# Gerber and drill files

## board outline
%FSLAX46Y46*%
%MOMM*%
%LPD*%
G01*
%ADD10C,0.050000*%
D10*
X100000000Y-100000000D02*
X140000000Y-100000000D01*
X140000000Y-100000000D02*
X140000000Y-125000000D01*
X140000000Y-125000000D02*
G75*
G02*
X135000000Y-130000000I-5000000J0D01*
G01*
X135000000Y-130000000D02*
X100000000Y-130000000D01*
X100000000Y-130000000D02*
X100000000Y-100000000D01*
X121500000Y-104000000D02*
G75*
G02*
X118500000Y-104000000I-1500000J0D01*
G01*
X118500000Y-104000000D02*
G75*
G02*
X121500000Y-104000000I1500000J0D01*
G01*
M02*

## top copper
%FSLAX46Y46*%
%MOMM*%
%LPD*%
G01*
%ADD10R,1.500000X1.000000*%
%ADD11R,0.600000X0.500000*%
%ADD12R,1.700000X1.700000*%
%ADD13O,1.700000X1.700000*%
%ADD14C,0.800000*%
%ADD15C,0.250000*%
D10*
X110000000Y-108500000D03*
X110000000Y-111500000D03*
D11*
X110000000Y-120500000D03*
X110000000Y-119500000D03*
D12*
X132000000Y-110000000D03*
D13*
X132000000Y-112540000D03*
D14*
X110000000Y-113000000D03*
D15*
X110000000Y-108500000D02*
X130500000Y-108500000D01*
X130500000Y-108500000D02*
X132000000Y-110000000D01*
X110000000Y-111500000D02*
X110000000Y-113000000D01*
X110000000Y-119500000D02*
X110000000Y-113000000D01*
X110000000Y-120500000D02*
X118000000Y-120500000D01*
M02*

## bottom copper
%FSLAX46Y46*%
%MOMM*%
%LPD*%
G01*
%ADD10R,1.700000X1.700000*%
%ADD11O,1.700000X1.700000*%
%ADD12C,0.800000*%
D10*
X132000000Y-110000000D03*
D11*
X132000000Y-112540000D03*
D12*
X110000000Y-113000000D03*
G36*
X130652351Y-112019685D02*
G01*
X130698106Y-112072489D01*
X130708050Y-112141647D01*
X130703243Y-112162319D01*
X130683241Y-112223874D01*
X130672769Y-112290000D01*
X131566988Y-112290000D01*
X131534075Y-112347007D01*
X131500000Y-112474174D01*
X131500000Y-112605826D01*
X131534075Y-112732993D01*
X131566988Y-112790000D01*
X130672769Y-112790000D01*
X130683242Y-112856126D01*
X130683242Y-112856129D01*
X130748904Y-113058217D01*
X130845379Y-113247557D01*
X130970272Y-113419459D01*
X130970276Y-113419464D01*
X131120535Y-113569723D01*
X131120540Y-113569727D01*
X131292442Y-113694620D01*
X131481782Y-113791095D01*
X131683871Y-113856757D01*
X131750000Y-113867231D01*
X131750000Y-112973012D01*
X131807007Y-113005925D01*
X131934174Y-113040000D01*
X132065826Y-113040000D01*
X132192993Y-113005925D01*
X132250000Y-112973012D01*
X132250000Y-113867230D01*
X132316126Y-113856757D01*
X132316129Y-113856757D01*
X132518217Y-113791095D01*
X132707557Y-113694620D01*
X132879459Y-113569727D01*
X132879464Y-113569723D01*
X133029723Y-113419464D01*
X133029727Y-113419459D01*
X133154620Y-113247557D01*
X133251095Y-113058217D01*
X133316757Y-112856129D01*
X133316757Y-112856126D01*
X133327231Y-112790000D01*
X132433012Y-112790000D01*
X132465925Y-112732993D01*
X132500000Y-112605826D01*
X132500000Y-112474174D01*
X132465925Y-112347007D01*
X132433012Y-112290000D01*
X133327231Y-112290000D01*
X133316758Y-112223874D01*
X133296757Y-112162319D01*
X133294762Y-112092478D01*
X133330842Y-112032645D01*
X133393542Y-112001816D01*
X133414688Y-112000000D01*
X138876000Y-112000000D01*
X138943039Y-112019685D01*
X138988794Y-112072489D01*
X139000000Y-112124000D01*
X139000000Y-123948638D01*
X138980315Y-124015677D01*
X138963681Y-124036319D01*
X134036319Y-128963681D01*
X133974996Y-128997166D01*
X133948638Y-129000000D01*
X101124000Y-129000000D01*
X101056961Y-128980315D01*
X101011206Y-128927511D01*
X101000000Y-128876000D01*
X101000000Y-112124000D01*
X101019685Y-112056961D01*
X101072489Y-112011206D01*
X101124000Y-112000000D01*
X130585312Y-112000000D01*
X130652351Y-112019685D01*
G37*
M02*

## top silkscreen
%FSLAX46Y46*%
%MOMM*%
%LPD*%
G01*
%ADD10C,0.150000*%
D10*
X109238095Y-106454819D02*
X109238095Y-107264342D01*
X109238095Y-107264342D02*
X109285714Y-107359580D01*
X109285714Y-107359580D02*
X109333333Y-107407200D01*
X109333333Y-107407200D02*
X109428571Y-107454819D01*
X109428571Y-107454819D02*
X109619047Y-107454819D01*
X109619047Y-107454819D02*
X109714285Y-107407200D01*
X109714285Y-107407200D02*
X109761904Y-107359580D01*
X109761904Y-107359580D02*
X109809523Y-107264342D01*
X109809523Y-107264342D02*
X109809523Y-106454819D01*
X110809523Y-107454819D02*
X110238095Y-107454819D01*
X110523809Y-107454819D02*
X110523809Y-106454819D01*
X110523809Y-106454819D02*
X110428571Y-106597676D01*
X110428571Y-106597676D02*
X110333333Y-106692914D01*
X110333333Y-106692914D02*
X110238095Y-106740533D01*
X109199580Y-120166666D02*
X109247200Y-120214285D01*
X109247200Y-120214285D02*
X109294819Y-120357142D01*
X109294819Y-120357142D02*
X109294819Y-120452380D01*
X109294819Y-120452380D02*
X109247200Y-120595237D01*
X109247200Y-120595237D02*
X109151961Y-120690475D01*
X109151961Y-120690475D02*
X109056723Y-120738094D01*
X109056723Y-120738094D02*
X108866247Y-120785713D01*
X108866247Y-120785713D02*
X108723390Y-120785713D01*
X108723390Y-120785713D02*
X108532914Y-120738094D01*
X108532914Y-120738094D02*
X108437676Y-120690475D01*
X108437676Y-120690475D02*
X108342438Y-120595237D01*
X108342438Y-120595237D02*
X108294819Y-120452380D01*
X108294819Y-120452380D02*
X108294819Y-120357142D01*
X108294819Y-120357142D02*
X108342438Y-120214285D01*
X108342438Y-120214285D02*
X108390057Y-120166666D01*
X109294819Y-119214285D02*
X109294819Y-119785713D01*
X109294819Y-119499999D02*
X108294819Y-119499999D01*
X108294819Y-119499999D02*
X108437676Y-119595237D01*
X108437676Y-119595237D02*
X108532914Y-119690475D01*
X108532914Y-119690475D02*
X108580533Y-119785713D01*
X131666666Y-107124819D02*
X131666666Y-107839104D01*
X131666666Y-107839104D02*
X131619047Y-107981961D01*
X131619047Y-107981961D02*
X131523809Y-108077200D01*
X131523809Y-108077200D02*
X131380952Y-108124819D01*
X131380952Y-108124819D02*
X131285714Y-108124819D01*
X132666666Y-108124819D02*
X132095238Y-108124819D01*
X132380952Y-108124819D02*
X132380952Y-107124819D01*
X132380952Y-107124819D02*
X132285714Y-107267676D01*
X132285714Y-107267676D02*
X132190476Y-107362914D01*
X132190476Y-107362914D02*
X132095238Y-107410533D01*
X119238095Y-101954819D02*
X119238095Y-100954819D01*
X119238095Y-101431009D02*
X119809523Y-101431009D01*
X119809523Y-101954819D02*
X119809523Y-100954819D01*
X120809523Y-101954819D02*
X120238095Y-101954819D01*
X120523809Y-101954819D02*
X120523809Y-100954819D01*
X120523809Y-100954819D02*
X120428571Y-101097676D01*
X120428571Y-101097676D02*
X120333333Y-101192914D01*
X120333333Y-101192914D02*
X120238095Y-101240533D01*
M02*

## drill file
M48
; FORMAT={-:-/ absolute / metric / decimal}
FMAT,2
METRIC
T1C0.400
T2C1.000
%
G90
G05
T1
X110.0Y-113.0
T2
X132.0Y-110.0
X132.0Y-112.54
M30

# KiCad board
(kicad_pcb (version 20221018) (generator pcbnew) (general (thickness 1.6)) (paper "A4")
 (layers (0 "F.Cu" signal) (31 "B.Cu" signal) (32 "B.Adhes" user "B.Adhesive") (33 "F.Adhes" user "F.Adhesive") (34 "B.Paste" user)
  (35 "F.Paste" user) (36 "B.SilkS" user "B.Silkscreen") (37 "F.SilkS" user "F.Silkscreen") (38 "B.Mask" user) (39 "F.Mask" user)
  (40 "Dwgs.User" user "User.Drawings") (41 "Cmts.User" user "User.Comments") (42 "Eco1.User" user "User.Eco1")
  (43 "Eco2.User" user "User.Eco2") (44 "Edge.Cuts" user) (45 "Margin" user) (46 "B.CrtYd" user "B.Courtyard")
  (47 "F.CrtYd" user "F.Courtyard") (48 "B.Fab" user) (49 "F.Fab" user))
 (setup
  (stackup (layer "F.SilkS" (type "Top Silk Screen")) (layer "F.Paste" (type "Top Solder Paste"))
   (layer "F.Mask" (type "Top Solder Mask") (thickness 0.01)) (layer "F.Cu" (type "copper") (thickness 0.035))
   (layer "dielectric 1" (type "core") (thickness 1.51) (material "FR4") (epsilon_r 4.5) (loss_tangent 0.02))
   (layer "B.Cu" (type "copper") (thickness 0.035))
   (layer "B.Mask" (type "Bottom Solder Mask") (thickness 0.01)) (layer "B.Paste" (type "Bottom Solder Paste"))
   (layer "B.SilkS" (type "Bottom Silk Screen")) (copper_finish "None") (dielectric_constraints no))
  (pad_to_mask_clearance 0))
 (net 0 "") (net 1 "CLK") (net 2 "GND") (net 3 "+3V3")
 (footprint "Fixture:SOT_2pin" (layer "F.Cu") (at 110 110)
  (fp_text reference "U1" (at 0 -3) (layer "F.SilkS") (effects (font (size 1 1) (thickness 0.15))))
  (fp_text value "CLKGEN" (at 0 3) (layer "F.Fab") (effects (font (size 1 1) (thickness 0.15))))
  (pad "1" smd rect (at 0 -1.5) (size 1.5 1) (layers "F.Cu" "F.Paste" "F.Mask") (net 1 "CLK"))
  (pad "2" smd rect (at 0 1.5) (size 1.5 1) (layers "F.Cu" "F.Paste" "F.Mask") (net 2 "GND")))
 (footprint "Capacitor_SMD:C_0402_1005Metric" (layer "F.Cu") (at 110 120 90)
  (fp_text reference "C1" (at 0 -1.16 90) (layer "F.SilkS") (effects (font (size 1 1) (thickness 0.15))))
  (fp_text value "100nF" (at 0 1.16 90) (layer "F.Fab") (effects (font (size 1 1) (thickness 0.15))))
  (pad "1" smd rect (at -0.5 0 90) (size 0.5 0.6) (layers "F.Cu" "F.Paste" "F.Mask") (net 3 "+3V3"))
  (pad "2" smd rect (at 0.5 0 90) (size 0.5 0.6) (layers "F.Cu" "F.Paste" "F.Mask") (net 2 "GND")))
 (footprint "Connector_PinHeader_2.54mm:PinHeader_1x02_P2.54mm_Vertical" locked (layer "F.Cu") (at 132 110)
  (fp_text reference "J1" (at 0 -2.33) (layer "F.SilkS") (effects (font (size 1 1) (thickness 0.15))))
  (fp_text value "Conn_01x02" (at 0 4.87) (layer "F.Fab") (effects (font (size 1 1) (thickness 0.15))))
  (pad "1" thru_hole rect (at 0 0) (size 1.7 1.7) (drill 1) (layers "*.Cu" "*.Mask") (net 1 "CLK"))
  (pad "2" thru_hole oval (at 0 2.54) (size 1.7 1.7) (drill 1) (layers "*.Cu" "*.Mask") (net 2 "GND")))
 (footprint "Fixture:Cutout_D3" (layer "F.Cu") (at 120 104)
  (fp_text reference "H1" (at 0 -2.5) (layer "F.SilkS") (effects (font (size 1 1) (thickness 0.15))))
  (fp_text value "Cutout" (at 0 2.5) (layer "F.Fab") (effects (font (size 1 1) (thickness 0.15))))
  (fp_circle (center 0 0) (end 1.5 0) (stroke (width 0.05) (type default)) (fill none) (layer "Edge.Cuts")))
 (gr_line (start 100 100) (end 140 100) (stroke (width 0.05) (type default)) (layer "Edge.Cuts"))
 (gr_line (start 140 100) (end 140 125) (stroke (width 0.05) (type default)) (layer "Edge.Cuts"))
 (gr_arc (start 140 125) (mid 138.535534 128.535534) (end 135 130) (stroke (width 0.05) (type default)) (layer "Edge.Cuts"))
 (gr_line (start 135 130) (end 100 130) (stroke (width 0.05) (type default)) (layer "Edge.Cuts"))
 (gr_line (start 100 130) (end 100 100) (stroke (width 0.05) (type default)) (layer "Edge.Cuts"))
 (segment (start 110 108.5) (end 130.5 108.5) (width 0.25) (layer "F.Cu") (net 1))
 (segment (start 130.5 108.5) (end 132 110) (width 0.25) (layer "F.Cu") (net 1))
 (segment (start 110 111.5) (end 110 113) (width 0.25) (layer "F.Cu") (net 2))
 (segment (start 110 119.5) (end 110 113) (width 0.25) (layer "F.Cu") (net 2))
 (segment (start 110 120.5) (end 118 120.5) (width 0.25) (layer "F.Cu") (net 3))
 (via (at 110 113) (size 0.8) (drill 0.4) (layers "F.Cu" "B.Cu") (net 2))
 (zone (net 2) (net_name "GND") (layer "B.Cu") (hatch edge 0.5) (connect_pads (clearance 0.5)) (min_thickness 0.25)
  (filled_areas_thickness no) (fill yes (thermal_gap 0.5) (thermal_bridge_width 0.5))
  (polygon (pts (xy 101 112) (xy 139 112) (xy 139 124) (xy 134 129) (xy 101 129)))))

